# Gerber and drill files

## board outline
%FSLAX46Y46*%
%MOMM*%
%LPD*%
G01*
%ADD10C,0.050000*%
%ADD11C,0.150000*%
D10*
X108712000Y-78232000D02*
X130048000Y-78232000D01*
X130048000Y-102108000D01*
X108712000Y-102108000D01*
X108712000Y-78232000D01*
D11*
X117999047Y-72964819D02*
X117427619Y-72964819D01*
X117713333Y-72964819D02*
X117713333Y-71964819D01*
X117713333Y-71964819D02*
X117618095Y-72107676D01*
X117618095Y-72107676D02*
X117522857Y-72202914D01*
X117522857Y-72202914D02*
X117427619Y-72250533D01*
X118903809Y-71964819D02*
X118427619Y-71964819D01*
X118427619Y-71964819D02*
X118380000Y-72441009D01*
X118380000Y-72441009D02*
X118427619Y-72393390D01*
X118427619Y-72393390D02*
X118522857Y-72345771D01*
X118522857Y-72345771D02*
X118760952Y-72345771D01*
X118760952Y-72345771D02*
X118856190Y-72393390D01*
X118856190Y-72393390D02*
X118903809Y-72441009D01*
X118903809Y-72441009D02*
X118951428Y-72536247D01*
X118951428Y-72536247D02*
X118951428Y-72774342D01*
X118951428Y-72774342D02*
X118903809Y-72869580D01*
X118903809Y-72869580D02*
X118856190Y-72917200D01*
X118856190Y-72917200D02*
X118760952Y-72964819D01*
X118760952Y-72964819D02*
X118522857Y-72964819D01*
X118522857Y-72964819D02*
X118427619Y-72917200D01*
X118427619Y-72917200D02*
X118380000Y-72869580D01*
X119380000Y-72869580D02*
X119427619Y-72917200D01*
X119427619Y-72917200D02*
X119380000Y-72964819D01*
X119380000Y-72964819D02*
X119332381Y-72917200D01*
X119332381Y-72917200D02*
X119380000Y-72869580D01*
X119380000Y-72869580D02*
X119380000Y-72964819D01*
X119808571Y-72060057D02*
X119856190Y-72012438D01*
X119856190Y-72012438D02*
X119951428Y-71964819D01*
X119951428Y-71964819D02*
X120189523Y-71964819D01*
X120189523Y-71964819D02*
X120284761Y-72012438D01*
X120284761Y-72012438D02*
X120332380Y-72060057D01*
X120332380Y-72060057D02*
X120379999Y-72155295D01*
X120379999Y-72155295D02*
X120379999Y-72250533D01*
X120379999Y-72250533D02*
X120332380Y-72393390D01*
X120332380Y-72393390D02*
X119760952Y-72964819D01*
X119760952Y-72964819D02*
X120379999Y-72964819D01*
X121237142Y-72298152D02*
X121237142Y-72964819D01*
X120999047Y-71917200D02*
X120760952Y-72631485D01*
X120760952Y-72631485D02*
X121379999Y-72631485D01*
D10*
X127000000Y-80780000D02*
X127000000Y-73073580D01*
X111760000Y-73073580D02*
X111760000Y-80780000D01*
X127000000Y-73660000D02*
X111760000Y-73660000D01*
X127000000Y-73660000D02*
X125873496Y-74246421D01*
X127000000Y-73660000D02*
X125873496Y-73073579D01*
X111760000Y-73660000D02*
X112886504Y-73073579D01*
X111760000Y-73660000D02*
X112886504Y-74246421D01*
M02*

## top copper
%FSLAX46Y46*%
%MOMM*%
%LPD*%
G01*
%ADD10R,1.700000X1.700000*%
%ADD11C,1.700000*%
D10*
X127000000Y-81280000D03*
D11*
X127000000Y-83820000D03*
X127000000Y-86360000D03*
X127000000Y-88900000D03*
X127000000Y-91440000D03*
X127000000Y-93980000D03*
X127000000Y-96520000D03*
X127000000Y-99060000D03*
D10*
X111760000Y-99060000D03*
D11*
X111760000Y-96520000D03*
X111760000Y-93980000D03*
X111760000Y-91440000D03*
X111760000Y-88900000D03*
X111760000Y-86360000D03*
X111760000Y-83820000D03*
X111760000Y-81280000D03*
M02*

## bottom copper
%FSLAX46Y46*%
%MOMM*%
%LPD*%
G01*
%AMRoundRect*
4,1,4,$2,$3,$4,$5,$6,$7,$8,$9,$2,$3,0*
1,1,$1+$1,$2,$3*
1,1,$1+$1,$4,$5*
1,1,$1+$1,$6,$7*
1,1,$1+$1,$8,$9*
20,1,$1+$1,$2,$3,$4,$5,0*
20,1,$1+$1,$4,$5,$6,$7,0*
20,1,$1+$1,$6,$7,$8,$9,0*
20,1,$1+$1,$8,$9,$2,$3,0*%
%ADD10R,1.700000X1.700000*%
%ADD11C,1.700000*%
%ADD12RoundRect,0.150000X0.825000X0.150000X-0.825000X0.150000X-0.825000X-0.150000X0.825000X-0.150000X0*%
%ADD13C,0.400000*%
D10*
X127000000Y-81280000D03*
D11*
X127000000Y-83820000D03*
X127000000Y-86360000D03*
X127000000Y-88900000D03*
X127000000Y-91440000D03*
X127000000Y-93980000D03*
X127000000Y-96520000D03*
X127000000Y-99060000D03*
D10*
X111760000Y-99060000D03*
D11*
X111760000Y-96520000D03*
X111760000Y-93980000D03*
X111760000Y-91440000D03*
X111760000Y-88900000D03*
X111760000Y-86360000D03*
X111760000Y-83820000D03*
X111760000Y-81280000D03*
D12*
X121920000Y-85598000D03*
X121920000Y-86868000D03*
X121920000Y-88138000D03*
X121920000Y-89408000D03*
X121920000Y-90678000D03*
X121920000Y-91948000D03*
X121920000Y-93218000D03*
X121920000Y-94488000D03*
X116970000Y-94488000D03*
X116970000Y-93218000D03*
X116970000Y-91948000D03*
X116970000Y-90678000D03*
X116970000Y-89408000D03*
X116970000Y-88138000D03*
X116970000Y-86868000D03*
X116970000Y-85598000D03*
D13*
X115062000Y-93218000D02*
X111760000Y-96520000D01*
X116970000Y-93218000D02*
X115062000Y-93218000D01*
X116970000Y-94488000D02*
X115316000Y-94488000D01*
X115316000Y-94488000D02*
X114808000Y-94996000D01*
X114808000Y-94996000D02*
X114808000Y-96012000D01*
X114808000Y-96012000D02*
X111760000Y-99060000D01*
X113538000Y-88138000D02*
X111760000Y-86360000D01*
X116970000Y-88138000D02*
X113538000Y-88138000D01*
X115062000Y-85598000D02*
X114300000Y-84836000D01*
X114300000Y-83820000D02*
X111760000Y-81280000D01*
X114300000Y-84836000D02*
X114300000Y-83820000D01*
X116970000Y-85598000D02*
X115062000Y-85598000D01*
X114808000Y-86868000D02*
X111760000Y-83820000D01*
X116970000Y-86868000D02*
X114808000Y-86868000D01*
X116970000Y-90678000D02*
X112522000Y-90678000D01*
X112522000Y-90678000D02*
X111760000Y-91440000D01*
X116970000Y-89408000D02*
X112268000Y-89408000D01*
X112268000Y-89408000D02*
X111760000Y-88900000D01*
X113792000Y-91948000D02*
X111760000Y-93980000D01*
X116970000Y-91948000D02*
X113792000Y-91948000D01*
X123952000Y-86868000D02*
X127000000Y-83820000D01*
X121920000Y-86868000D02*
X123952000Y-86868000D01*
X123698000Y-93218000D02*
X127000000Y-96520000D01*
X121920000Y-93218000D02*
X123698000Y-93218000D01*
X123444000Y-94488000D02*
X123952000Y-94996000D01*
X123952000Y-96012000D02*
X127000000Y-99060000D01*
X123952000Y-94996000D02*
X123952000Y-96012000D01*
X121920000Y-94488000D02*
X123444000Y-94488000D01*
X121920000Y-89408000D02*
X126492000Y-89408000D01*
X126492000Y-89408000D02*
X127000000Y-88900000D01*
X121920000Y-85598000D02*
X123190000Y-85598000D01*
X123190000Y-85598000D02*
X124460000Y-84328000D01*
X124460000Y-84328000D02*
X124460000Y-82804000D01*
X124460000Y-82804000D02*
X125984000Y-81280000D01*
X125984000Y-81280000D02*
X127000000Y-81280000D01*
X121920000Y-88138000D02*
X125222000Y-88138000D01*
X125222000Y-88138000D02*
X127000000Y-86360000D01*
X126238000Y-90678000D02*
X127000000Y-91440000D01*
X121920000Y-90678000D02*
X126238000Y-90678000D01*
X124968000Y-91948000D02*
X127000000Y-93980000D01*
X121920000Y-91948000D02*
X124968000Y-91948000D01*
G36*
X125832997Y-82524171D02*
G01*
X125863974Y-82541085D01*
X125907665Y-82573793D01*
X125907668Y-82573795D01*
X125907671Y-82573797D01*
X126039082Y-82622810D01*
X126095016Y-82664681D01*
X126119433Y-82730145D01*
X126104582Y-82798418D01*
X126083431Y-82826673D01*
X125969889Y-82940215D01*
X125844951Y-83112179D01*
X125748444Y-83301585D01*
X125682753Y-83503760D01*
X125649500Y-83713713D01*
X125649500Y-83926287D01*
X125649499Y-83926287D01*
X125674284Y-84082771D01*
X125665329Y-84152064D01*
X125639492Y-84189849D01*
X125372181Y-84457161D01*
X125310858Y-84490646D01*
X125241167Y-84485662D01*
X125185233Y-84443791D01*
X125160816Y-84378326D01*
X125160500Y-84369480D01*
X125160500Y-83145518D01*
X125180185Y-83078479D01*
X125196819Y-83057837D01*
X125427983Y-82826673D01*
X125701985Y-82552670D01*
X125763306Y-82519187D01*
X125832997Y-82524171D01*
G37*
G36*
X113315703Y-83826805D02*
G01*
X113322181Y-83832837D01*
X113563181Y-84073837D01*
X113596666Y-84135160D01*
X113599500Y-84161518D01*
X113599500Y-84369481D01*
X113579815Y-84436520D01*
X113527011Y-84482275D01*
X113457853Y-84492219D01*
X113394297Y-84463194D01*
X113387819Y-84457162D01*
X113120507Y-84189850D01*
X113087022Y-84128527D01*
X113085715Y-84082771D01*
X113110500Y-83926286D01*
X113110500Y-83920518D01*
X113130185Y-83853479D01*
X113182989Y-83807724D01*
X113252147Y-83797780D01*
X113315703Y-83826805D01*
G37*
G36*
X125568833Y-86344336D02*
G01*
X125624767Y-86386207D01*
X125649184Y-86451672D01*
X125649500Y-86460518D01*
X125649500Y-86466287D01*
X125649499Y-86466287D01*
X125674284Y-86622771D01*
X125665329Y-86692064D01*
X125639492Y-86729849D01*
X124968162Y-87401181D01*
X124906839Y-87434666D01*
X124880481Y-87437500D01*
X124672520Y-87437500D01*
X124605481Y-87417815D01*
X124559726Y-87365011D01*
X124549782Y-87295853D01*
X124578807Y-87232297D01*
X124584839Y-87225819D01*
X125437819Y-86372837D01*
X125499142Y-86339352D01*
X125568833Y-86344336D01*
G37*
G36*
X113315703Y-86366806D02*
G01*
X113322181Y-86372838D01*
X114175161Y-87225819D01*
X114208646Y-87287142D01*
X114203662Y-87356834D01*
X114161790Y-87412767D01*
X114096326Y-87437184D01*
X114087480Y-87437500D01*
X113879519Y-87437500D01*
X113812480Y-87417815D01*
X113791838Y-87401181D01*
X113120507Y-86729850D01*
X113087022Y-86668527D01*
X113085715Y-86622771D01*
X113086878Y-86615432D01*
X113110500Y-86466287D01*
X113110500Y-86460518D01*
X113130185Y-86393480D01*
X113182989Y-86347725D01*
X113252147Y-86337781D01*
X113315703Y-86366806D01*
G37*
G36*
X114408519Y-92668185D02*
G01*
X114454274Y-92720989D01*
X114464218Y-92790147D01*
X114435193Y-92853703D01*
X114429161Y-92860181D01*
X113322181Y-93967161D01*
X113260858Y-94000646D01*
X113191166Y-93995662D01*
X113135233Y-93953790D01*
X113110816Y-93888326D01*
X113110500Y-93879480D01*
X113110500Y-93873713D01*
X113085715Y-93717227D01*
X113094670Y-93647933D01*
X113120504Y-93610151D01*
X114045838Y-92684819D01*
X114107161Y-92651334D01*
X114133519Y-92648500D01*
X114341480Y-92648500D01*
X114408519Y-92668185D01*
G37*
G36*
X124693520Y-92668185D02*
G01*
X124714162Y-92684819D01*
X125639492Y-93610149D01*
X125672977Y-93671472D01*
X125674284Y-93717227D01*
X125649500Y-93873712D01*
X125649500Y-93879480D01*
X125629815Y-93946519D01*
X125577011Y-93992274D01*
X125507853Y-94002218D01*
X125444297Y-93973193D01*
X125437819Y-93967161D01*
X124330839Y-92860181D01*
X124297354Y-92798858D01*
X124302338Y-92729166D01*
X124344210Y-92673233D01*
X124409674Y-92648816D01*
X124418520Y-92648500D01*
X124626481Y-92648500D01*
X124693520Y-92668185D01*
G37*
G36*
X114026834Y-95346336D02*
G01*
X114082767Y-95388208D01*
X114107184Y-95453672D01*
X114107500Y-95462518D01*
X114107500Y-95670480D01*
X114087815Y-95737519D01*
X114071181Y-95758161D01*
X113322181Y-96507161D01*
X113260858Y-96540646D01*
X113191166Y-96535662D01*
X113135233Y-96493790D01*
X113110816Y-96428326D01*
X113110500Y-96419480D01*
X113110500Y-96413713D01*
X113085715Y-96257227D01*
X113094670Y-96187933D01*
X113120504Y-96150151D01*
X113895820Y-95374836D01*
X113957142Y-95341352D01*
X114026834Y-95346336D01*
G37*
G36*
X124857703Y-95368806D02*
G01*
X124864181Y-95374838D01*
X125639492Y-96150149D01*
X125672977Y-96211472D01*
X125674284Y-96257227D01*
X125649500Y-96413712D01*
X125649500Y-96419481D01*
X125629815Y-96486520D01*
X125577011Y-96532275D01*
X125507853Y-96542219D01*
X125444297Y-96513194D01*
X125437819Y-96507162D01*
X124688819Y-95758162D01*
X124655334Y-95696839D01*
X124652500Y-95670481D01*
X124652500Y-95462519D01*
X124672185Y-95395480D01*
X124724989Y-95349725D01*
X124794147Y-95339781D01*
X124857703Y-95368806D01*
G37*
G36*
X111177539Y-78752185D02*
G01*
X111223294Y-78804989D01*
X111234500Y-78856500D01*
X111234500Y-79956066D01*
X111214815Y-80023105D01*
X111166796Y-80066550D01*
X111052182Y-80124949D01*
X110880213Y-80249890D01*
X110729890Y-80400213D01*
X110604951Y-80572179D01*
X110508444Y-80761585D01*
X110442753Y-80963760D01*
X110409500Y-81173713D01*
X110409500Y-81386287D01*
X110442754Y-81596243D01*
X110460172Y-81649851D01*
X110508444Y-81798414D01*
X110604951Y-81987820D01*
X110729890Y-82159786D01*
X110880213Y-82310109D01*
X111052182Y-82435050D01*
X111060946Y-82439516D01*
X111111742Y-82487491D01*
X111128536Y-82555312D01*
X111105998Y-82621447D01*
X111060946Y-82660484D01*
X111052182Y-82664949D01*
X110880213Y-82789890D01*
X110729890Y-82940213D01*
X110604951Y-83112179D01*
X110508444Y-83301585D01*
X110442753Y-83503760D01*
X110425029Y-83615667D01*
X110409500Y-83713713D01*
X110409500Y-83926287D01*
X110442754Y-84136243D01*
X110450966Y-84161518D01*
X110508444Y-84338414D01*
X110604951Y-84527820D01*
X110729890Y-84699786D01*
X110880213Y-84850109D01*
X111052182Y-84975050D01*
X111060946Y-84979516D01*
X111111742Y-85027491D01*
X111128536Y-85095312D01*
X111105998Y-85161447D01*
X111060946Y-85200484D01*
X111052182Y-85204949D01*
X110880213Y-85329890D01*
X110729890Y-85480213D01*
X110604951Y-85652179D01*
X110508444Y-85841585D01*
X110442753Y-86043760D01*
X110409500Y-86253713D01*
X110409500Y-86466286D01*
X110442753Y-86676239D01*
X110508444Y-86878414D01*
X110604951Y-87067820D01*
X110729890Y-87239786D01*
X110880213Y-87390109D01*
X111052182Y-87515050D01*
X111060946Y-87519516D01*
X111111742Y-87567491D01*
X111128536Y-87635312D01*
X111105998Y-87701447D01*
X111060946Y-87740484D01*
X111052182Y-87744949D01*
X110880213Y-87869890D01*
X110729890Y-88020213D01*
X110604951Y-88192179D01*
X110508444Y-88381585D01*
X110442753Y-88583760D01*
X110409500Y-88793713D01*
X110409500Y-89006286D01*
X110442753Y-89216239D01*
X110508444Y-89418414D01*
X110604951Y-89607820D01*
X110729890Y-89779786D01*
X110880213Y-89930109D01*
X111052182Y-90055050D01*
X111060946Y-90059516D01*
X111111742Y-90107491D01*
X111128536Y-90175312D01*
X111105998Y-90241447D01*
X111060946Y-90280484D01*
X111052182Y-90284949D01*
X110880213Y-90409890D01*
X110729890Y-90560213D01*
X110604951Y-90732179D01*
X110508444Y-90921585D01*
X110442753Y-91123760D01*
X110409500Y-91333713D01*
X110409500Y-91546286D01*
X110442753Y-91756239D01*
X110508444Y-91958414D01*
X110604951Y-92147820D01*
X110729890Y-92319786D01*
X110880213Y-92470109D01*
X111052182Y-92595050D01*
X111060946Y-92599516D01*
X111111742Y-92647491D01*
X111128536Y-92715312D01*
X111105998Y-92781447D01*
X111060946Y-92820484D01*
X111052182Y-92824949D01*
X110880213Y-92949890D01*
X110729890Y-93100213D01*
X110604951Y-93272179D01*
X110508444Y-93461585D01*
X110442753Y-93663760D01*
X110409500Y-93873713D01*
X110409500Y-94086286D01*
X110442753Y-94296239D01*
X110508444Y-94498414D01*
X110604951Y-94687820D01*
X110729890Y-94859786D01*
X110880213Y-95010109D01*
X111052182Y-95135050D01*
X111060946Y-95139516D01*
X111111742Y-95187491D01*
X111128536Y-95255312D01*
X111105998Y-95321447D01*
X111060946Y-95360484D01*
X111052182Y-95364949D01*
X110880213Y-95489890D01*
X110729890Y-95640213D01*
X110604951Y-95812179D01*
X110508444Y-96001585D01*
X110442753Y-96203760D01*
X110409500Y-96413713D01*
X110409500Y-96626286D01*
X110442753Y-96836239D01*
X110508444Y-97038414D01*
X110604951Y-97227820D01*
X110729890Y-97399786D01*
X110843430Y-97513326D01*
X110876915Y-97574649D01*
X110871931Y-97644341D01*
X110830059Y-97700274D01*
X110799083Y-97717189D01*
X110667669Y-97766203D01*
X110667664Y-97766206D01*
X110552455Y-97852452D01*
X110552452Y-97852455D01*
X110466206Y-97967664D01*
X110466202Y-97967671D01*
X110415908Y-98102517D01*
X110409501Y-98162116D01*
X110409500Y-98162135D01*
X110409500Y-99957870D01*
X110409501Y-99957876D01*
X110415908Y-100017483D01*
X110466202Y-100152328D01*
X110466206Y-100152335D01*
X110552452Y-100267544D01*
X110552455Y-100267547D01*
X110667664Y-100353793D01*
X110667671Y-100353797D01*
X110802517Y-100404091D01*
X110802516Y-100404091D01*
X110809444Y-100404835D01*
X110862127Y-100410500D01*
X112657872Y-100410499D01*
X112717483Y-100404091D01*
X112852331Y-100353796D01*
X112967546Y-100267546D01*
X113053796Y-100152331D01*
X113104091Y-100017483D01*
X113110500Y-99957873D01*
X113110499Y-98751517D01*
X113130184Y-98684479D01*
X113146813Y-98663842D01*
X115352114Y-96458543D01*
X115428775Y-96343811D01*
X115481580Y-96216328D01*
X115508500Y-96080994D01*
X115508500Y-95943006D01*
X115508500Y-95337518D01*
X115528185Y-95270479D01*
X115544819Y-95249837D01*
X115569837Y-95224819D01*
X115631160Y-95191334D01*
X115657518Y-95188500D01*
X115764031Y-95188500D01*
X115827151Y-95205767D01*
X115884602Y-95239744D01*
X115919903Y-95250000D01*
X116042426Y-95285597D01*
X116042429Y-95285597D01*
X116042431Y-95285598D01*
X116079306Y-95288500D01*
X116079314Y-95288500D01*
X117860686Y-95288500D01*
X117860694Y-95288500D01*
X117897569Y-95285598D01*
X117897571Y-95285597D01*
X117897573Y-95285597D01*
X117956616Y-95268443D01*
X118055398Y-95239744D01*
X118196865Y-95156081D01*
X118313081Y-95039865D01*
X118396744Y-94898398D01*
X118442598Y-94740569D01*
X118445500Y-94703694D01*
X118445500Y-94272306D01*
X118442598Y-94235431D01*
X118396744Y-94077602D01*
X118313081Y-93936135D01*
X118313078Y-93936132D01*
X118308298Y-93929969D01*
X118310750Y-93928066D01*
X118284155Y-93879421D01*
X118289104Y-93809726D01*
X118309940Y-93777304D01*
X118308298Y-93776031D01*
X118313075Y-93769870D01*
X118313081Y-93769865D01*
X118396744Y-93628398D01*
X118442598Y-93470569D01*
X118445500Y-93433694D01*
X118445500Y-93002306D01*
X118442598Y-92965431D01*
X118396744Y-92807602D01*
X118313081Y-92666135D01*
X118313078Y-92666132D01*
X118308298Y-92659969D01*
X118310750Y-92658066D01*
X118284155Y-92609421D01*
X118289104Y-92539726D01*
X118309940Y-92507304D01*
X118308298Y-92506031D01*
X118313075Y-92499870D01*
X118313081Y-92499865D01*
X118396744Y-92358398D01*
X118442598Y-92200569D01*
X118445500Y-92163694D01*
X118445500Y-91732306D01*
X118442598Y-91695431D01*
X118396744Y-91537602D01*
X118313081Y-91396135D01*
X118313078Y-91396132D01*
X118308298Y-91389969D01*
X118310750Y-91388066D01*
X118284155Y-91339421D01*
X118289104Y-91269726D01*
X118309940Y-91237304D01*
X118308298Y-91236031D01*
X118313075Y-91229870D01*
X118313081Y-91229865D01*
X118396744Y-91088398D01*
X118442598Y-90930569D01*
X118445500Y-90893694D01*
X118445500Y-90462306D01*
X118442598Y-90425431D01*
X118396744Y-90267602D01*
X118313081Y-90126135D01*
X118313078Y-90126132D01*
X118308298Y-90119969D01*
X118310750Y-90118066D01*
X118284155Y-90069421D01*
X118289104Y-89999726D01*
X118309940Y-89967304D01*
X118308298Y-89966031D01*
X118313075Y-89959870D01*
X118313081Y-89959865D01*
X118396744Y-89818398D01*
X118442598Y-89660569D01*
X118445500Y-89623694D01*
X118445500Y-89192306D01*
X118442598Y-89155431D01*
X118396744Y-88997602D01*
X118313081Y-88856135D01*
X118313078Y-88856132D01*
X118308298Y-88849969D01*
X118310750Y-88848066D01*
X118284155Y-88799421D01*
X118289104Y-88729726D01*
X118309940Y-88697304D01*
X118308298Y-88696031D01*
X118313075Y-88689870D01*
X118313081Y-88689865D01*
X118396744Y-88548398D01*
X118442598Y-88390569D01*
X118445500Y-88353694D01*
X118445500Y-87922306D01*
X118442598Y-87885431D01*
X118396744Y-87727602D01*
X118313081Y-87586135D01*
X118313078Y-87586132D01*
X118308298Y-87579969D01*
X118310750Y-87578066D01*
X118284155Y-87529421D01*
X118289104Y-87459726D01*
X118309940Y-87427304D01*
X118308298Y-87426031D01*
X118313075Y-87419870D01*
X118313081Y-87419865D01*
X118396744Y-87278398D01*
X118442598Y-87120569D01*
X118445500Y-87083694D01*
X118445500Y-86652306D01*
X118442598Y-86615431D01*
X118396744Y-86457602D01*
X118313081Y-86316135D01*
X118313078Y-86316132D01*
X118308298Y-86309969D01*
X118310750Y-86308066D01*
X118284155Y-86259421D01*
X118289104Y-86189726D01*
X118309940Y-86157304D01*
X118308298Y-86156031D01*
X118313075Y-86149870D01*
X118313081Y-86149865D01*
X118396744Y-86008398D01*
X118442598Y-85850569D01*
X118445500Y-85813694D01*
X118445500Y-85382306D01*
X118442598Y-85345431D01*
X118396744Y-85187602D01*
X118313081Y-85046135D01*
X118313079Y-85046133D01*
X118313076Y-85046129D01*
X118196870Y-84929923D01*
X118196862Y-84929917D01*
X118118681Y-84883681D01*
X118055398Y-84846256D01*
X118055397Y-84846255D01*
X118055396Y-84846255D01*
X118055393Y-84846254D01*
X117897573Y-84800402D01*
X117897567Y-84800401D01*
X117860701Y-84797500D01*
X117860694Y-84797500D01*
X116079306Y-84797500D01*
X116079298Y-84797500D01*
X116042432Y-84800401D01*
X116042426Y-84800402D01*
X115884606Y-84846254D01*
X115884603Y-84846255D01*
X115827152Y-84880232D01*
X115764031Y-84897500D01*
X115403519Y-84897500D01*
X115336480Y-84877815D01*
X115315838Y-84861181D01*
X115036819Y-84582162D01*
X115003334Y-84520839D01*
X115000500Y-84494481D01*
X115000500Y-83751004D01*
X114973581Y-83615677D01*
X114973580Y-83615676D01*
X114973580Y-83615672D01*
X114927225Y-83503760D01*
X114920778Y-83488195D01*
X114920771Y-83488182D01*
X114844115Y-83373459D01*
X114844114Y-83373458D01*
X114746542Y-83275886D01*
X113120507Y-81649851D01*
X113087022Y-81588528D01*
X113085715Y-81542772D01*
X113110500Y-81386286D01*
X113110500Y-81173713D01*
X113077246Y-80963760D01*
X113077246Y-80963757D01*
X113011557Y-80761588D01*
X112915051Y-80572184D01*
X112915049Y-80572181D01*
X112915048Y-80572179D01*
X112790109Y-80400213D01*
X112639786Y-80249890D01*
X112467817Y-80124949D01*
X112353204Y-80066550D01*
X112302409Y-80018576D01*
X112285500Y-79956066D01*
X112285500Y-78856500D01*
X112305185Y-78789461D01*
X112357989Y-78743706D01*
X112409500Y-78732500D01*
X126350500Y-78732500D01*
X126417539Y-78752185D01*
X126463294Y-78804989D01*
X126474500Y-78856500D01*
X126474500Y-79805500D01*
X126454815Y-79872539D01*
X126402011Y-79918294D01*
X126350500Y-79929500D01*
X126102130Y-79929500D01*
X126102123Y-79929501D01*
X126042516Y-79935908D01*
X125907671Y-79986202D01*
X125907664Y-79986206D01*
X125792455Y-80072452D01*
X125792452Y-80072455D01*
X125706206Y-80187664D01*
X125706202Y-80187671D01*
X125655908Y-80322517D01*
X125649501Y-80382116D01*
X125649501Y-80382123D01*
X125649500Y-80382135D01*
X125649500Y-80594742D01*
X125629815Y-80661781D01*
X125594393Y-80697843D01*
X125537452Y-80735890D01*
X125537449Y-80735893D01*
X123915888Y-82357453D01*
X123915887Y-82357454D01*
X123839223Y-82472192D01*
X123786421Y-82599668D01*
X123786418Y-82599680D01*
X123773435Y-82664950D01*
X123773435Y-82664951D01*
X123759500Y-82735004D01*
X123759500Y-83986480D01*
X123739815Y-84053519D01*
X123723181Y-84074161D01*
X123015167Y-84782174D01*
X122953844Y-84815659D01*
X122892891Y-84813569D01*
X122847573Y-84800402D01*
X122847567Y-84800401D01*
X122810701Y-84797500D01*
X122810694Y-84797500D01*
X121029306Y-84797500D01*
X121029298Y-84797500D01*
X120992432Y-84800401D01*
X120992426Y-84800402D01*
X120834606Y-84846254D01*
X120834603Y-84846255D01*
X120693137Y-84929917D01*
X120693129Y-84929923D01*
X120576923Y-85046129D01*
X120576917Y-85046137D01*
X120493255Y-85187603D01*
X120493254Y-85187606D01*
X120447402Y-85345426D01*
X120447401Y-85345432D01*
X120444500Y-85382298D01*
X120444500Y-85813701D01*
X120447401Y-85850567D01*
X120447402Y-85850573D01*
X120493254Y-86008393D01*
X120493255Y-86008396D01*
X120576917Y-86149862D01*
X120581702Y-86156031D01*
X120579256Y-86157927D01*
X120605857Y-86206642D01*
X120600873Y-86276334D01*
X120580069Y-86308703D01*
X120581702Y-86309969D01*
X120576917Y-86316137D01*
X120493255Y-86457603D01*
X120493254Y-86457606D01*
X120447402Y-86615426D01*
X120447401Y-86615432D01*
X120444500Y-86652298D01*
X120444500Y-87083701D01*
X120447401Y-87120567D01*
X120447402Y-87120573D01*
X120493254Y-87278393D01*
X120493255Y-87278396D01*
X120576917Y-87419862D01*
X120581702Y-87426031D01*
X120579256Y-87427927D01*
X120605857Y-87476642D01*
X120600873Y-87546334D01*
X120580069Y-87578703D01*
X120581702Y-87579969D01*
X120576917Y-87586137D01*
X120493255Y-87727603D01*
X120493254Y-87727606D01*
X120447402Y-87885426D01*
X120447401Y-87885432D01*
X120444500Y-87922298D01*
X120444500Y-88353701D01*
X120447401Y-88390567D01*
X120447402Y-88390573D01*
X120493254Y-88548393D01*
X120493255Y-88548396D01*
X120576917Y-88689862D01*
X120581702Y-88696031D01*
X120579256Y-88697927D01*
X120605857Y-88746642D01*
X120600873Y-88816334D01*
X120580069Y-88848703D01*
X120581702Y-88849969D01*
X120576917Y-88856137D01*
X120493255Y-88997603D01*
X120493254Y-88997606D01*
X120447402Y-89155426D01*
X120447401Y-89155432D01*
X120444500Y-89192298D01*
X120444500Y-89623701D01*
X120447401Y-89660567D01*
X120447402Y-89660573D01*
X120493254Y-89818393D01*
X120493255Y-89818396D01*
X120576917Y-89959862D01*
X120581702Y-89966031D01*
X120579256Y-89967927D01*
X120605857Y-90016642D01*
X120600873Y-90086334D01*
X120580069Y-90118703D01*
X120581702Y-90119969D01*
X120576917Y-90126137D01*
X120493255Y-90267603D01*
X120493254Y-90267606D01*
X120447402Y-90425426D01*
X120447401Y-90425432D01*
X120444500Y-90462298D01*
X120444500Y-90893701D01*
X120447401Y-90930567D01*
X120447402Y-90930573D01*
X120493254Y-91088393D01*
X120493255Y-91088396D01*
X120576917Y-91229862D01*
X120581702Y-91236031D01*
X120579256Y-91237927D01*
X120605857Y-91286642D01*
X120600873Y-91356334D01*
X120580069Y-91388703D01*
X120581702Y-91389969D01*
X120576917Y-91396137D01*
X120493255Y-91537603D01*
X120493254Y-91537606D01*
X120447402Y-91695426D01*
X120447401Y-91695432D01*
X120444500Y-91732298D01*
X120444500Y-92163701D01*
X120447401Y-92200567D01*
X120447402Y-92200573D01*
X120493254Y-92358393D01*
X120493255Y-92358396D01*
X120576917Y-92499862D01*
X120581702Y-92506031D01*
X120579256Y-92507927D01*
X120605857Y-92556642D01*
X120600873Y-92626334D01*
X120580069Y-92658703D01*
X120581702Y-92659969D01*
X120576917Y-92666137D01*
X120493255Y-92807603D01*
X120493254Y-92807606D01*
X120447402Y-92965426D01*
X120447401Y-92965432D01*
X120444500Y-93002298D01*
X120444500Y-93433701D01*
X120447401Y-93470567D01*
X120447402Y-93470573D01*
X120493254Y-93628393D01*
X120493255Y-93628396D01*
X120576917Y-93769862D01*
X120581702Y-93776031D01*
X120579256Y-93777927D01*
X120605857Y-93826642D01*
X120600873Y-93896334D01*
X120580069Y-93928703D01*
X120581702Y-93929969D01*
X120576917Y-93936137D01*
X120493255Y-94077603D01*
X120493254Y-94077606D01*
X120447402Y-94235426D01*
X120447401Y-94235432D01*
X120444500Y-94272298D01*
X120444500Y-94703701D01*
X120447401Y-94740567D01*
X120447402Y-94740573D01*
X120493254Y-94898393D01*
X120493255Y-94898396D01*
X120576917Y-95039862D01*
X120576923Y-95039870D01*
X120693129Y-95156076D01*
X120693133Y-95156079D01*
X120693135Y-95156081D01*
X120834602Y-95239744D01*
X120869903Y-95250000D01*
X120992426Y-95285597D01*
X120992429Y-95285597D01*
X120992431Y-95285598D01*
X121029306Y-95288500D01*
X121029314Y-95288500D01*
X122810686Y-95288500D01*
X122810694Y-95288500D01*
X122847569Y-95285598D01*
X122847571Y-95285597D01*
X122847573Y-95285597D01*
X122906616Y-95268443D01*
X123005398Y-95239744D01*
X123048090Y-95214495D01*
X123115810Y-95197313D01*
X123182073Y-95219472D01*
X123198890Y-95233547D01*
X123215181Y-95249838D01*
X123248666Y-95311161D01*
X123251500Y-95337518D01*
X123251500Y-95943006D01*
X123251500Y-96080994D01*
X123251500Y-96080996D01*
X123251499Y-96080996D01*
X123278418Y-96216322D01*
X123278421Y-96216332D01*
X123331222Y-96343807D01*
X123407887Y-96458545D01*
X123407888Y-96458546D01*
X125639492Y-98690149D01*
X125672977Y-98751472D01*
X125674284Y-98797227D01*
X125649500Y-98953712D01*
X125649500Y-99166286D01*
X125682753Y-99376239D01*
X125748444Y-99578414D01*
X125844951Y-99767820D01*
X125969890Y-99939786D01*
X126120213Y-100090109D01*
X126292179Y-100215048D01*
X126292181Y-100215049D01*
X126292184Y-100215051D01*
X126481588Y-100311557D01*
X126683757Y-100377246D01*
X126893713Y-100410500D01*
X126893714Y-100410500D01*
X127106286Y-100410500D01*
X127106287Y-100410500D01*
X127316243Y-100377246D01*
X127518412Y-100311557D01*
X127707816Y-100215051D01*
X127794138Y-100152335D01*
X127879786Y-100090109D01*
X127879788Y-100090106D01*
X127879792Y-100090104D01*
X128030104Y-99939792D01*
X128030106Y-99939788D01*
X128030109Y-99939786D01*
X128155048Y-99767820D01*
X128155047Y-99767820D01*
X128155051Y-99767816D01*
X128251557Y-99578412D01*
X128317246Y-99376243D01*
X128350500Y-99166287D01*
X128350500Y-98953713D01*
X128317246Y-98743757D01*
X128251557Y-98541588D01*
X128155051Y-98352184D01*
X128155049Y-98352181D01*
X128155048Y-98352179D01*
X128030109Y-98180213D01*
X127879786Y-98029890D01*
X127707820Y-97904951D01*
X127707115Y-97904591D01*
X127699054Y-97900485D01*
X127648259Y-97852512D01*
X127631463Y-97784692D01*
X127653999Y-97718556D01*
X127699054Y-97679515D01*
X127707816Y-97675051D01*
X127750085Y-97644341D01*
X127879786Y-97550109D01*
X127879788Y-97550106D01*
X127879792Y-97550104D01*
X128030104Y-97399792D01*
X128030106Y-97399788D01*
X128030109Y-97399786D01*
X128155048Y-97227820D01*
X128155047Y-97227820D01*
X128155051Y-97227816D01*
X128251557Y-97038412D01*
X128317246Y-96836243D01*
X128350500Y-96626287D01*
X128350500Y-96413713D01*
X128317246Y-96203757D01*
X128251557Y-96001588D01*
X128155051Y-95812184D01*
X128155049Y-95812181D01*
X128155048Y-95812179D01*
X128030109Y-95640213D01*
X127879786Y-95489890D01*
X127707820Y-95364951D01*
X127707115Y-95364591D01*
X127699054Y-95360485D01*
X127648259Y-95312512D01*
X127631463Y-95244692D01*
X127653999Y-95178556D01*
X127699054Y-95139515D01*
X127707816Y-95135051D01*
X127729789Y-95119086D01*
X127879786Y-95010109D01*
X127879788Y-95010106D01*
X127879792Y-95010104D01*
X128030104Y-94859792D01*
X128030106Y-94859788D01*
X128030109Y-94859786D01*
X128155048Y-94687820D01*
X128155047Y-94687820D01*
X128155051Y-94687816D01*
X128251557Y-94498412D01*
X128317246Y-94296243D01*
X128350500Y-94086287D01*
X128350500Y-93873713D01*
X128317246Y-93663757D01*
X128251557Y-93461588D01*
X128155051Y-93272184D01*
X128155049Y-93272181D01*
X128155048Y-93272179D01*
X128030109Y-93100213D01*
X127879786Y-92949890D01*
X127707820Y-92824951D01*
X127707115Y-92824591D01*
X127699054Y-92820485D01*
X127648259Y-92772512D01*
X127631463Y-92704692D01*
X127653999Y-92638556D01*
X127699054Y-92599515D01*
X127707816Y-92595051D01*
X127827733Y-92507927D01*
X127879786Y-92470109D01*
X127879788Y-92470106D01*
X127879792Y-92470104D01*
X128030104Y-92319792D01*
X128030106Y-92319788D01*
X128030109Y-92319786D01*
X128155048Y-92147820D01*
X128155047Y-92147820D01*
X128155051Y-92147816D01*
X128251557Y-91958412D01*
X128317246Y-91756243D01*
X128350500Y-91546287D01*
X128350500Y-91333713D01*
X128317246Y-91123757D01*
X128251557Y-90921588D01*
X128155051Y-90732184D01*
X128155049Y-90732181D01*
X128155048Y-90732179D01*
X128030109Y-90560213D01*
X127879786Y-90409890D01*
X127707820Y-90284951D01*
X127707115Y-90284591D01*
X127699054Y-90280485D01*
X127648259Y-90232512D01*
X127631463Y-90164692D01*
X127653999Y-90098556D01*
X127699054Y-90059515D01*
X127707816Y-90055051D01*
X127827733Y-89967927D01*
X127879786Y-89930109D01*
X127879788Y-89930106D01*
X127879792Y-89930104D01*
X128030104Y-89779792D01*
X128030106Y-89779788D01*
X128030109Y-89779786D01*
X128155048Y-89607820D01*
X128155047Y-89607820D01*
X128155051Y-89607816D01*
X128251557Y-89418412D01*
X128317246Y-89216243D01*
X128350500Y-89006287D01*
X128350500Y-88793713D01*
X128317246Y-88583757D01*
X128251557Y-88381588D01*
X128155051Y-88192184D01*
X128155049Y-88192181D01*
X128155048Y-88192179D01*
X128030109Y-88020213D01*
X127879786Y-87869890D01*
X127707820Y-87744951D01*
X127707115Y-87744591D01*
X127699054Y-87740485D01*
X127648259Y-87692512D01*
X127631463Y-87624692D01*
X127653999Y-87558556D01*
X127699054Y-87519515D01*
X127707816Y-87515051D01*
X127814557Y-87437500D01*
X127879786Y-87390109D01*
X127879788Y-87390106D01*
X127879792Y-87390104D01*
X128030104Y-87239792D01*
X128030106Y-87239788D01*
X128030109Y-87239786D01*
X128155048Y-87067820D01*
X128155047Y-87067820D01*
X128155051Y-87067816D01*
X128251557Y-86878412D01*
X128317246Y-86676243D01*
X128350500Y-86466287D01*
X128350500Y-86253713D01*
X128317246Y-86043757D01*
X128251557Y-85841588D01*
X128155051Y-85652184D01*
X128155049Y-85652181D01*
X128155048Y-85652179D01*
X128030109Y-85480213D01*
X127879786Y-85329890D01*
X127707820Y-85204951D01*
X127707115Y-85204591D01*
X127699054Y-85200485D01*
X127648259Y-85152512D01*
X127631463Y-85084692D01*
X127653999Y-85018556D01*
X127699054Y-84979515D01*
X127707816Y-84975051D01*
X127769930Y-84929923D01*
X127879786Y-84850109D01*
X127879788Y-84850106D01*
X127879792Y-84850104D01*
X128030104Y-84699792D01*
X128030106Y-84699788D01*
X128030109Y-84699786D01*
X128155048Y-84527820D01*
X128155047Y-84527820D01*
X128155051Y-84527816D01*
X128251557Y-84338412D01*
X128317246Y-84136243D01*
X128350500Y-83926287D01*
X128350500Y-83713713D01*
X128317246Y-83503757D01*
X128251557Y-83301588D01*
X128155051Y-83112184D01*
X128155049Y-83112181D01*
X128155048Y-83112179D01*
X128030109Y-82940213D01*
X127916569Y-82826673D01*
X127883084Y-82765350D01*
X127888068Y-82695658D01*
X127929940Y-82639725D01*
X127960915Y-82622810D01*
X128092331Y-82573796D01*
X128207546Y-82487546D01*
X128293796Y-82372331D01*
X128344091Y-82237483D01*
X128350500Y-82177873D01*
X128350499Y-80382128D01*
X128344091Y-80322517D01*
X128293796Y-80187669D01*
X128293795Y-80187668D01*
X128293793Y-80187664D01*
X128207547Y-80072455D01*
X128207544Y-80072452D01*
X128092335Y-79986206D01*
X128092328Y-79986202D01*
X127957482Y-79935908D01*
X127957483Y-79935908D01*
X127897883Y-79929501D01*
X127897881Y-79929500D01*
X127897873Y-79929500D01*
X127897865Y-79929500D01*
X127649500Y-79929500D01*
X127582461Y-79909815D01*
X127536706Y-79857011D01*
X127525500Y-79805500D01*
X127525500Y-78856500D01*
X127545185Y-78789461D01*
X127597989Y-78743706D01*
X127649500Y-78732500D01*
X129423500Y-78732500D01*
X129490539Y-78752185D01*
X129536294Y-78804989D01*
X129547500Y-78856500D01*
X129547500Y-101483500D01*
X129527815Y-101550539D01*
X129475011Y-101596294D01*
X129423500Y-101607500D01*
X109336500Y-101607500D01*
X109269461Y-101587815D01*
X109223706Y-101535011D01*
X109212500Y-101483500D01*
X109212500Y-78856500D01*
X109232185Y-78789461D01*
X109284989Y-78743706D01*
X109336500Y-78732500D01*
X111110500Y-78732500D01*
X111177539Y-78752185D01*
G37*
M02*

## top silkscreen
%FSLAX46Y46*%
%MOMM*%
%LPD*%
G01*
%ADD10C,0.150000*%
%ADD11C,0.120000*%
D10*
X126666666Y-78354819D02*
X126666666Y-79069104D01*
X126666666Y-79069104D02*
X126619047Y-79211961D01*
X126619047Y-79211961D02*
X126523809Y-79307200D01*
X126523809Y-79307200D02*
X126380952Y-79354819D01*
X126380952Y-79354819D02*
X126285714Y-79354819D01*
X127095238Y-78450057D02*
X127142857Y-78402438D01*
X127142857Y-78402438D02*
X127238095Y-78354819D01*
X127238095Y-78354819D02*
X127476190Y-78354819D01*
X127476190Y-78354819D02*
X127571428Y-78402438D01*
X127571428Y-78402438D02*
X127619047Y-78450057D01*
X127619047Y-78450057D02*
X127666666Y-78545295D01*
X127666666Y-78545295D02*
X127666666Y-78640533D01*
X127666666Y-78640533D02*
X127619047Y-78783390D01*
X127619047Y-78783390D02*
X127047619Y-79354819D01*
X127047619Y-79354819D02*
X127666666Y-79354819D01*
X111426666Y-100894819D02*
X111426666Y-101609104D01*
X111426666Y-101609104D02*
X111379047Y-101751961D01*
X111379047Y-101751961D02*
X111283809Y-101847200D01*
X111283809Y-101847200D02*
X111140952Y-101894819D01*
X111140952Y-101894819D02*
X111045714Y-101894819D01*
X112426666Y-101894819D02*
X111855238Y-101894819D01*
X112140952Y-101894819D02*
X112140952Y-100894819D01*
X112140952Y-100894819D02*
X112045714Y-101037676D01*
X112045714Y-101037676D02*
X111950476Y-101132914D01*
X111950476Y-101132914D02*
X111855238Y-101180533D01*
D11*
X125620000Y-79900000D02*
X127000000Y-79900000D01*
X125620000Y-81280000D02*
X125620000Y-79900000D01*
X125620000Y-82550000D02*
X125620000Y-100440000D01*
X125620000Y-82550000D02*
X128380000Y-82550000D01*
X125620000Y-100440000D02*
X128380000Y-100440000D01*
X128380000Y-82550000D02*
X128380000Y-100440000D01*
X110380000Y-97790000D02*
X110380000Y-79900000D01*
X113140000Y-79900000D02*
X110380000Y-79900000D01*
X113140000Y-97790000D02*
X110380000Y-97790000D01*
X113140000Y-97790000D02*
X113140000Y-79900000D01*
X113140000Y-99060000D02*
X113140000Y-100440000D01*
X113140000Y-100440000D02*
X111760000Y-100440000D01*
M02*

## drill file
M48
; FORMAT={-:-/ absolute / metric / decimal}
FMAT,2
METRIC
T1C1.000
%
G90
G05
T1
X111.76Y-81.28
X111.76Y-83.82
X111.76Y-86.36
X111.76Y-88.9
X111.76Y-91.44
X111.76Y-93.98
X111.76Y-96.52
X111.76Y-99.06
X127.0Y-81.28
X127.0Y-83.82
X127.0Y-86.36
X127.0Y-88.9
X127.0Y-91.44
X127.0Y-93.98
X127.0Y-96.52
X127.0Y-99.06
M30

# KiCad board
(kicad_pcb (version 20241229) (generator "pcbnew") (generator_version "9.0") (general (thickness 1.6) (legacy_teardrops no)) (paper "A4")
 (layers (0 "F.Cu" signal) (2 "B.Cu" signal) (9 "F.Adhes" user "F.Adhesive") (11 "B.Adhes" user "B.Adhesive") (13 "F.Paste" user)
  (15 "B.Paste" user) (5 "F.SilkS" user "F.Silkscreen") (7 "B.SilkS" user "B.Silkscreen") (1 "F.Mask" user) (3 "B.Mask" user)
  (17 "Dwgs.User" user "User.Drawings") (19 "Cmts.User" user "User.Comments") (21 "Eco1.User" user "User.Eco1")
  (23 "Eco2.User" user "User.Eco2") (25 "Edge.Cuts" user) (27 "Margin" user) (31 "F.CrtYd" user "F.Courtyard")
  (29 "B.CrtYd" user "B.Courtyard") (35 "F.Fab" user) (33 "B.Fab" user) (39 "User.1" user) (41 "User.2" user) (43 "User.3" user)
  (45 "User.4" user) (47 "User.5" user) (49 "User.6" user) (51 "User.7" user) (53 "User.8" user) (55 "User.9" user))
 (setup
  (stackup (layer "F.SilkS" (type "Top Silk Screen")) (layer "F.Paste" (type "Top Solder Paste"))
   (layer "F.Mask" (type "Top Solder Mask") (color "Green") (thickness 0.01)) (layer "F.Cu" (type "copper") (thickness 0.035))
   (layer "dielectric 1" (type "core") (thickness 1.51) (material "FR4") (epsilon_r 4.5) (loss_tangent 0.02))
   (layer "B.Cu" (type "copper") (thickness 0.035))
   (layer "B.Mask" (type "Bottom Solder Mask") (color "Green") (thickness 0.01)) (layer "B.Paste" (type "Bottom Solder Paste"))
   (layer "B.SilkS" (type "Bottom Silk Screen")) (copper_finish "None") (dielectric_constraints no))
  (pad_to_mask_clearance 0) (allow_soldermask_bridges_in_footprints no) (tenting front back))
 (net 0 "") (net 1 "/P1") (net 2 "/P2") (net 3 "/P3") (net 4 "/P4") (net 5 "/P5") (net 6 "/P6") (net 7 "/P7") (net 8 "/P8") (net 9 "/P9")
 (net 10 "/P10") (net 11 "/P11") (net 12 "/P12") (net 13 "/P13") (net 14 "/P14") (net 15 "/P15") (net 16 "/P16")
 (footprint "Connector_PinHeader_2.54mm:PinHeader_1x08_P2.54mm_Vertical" (layer "F.Cu") (at 127 81.28)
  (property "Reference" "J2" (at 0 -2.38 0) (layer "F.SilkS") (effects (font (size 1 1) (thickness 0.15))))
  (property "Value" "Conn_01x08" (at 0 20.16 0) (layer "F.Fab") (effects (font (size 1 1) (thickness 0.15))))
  (fp_line (start -1.38 -1.38) (end 0 -1.38) (stroke (width 0.12) (type solid)) (layer "F.SilkS"))
  (fp_line (start -1.38 0) (end -1.38 -1.38) (stroke (width 0.12) (type solid)) (layer "F.SilkS"))
  (fp_line (start -1.38 1.27) (end -1.38 19.16) (stroke (width 0.12) (type solid)) (layer "F.SilkS"))
  (fp_line (start -1.38 1.27) (end 1.38 1.27) (stroke (width 0.12) (type solid)) (layer "F.SilkS"))
  (fp_line (start -1.38 19.16) (end 1.38 19.16) (stroke (width 0.12) (type solid)) (layer "F.SilkS"))
  (fp_line (start 1.38 1.27) (end 1.38 19.16) (stroke (width 0.12) (type solid)) (layer "F.SilkS"))
  (pad "1" thru_hole rect (at 0 0) (size 1.7 1.7) (drill 1) (layers "*.Cu" "*.Mask") (remove_unused_layers no) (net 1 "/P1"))
  (pad "2" thru_hole circle (at 0 2.54) (size 1.7 1.7) (drill 1) (layers "*.Cu" "*.Mask") (remove_unused_layers no) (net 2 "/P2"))
  (pad "3" thru_hole circle (at 0 5.08) (size 1.7 1.7) (drill 1) (layers "*.Cu" "*.Mask") (remove_unused_layers no) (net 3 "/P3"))
  (pad "4" thru_hole circle (at 0 7.62) (size 1.7 1.7) (drill 1) (layers "*.Cu" "*.Mask") (remove_unused_layers no) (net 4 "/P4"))
  (pad "5" thru_hole circle (at 0 10.16) (size 1.7 1.7) (drill 1) (layers "*.Cu" "*.Mask") (remove_unused_layers no) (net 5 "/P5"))
  (pad "6" thru_hole circle (at 0 12.7) (size 1.7 1.7) (drill 1) (layers "*.Cu" "*.Mask") (remove_unused_layers no) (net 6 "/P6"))
  (pad "7" thru_hole circle (at 0 15.24) (size 1.7 1.7) (drill 1) (layers "*.Cu" "*.Mask") (remove_unused_layers no) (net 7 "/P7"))
  (pad "8" thru_hole circle (at 0 17.78) (size 1.7 1.7) (drill 1) (layers "*.Cu" "*.Mask") (remove_unused_layers no) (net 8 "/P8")))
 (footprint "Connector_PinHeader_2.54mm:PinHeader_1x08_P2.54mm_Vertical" (layer "F.Cu") (at 111.76 99.06 180)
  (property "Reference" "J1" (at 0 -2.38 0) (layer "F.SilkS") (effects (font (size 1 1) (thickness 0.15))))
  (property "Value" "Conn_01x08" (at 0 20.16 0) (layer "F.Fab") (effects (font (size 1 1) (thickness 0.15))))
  (fp_line (start 1.38 1.27) (end 1.38 19.16) (stroke (width 0.12) (type solid)) (layer "F.SilkS"))
  (fp_line (start -1.38 19.16) (end 1.38 19.16) (stroke (width 0.12) (type solid)) (layer "F.SilkS"))
  (fp_line (start -1.38 1.27) (end 1.38 1.27) (stroke (width 0.12) (type solid)) (layer "F.SilkS"))
  (fp_line (start -1.38 1.27) (end -1.38 19.16) (stroke (width 0.12) (type solid)) (layer "F.SilkS"))
  (fp_line (start -1.38 0) (end -1.38 -1.38) (stroke (width 0.12) (type solid)) (layer "F.SilkS"))
  (fp_line (start -1.38 -1.38) (end 0 -1.38) (stroke (width 0.12) (type solid)) (layer "F.SilkS"))
  (pad "1" thru_hole rect (at 0 0 180) (size 1.7 1.7) (drill 1) (layers "*.Cu" "*.Mask") (remove_unused_layers no) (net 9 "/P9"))
  (pad "2" thru_hole circle (at 0 2.54 180) (size 1.7 1.7) (drill 1) (layers "*.Cu" "*.Mask") (remove_unused_layers no) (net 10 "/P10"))
  (pad "3" thru_hole circle (at 0 5.08 180) (size 1.7 1.7) (drill 1) (layers "*.Cu" "*.Mask") (remove_unused_layers no) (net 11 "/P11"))
  (pad "4" thru_hole circle (at 0 7.62 180) (size 1.7 1.7) (drill 1) (layers "*.Cu" "*.Mask") (remove_unused_layers no) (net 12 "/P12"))
  (pad "5" thru_hole circle (at 0 10.16 180) (size 1.7 1.7) (drill 1) (layers "*.Cu" "*.Mask") (remove_unused_layers no) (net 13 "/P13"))
  (pad "6" thru_hole circle (at 0 12.7 180) (size 1.7 1.7) (drill 1) (layers "*.Cu" "*.Mask") (remove_unused_layers no) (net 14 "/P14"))
  (pad "7" thru_hole circle (at 0 15.24 180) (size 1.7 1.7) (drill 1) (layers "*.Cu" "*.Mask") (remove_unused_layers no) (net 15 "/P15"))
  (pad "8" thru_hole circle (at 0 17.78 180) (size 1.7 1.7) (drill 1) (layers "*.Cu" "*.Mask") (remove_unused_layers no) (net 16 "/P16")))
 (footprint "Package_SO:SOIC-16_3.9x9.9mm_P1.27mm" (layer "B.Cu") (at 119.445 90.043 180)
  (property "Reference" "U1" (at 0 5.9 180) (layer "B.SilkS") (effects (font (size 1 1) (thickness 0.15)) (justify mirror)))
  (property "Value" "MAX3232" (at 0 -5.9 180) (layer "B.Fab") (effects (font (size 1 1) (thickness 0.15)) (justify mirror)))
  (pad "1" smd roundrect (at -2.475 4.445 180) (size 1.95 0.6) (layers "B.Cu" "B.Mask" "B.Paste") (roundrect_rratio 0.25) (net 1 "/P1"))
  (pad "2" smd roundrect (at -2.475 3.175 180) (size 1.95 0.6) (layers "B.Cu" "B.Mask" "B.Paste") (roundrect_rratio 0.25) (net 2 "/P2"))
  (pad "3" smd roundrect (at -2.475 1.905 180) (size 1.95 0.6) (layers "B.Cu" "B.Mask" "B.Paste") (roundrect_rratio 0.25) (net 3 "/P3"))
  (pad "4" smd roundrect (at -2.475 0.635 180) (size 1.95 0.6) (layers "B.Cu" "B.Mask" "B.Paste") (roundrect_rratio 0.25) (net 4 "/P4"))
  (pad "5" smd roundrect (at -2.475 -0.635 180) (size 1.95 0.6) (layers "B.Cu" "B.Mask" "B.Paste") (roundrect_rratio 0.25) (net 5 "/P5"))
  (pad "6" smd roundrect (at -2.475 -1.905 180) (size 1.95 0.6) (layers "B.Cu" "B.Mask" "B.Paste") (roundrect_rratio 0.25) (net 6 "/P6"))
  (pad "7" smd roundrect (at -2.475 -3.175 180) (size 1.95 0.6) (layers "B.Cu" "B.Mask" "B.Paste") (roundrect_rratio 0.25) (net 7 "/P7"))
  (pad "8" smd roundrect (at -2.475 -4.445 180) (size 1.95 0.6) (layers "B.Cu" "B.Mask" "B.Paste") (roundrect_rratio 0.25) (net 8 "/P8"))
  (pad "9" smd roundrect (at 2.475 -4.445 180) (size 1.95 0.6) (layers "B.Cu" "B.Mask" "B.Paste") (roundrect_rratio 0.25) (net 9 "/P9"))
  (pad "10" smd roundrect (at 2.475 -3.175 180) (size 1.95 0.6) (layers "B.Cu" "B.Mask" "B.Paste") (roundrect_rratio 0.25) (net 10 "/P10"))
  (pad "11" smd roundrect (at 2.475 -1.905 180) (size 1.95 0.6) (layers "B.Cu" "B.Mask" "B.Paste") (roundrect_rratio 0.25) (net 11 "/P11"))
  (pad "12" smd roundrect (at 2.475 -0.635 180) (size 1.95 0.6) (layers "B.Cu" "B.Mask" "B.Paste") (roundrect_rratio 0.25) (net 12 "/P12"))
  (pad "13" smd roundrect (at 2.475 0.635 180) (size 1.95 0.6) (layers "B.Cu" "B.Mask" "B.Paste") (roundrect_rratio 0.25) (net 13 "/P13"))
  (pad "14" smd roundrect (at 2.475 1.905 180) (size 1.95 0.6) (layers "B.Cu" "B.Mask" "B.Paste") (roundrect_rratio 0.25) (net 14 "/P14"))
  (pad "15" smd roundrect (at 2.475 3.175 180) (size 1.95 0.6) (layers "B.Cu" "B.Mask" "B.Paste") (roundrect_rratio 0.25) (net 15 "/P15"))
  (pad "16" smd roundrect (at 2.475 4.445 180) (size 1.95 0.6) (layers "B.Cu" "B.Mask" "B.Paste") (roundrect_rratio 0.25) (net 16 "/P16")))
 (gr_rect (start 108.712 78.232) (end 130.048 102.108) (stroke (width 0.05) (type default)) (fill no) (layer "Edge.Cuts"))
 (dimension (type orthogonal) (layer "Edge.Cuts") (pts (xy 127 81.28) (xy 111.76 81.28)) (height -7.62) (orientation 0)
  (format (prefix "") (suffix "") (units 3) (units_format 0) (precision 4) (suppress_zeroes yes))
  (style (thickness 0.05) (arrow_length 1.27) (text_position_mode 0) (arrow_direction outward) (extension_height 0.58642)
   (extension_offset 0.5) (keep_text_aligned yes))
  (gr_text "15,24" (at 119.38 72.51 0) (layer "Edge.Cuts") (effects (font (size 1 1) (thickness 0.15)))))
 (segment (start 115.062 93.218) (end 111.76 96.52) (width 0.4) (layer "B.Cu") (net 10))
 (segment (start 116.97 93.218) (end 115.062 93.218) (width 0.4) (layer "B.Cu") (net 10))
 (segment (start 116.97 94.488) (end 115.316 94.488) (width 0.4) (layer "B.Cu") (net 9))
 (segment (start 115.316 94.488) (end 114.808 94.996) (width 0.4) (layer "B.Cu") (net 9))
 (segment (start 114.808 94.996) (end 114.808 96.012) (width 0.4) (layer "B.Cu") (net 9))
 (segment (start 114.808 96.012) (end 111.76 99.06) (width 0.4) (layer "B.Cu") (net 9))
 (segment (start 113.538 88.138) (end 111.76 86.36) (width 0.4) (layer "B.Cu") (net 14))
 (segment (start 116.97 88.138) (end 113.538 88.138) (width 0.4) (layer "B.Cu") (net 14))
 (segment (start 115.062 85.598) (end 114.3 84.836) (width 0.4) (layer "B.Cu") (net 16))
 (segment (start 114.3 83.82) (end 111.76 81.28) (width 0.4) (layer "B.Cu") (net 16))
 (segment (start 114.3 84.836) (end 114.3 83.82) (width 0.4) (layer "B.Cu") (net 16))
 (segment (start 116.97 85.598) (end 115.062 85.598) (width 0.4) (layer "B.Cu") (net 16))
 (segment (start 114.808 86.868) (end 111.76 83.82) (width 0.4) (layer "B.Cu") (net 15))
 (segment (start 116.97 86.868) (end 114.808 86.868) (width 0.4) (layer "B.Cu") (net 15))
 (segment (start 116.97 90.678) (end 112.522 90.678) (width 0.4) (layer "B.Cu") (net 12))
 (segment (start 112.522 90.678) (end 111.76 91.44) (width 0.4) (layer "B.Cu") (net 12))
 (segment (start 116.97 89.408) (end 112.268 89.408) (width 0.4) (layer "B.Cu") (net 13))
 (segment (start 112.268 89.408) (end 111.76 88.9) (width 0.4) (layer "B.Cu") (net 13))
 (segment (start 113.792 91.948) (end 111.76 93.98) (width 0.4) (layer "B.Cu") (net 11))
 (segment (start 116.97 91.948) (end 113.792 91.948) (width 0.4) (layer "B.Cu") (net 11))
 (segment (start 123.952 86.868) (end 127 83.82) (width 0.4) (layer "B.Cu") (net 2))
 (segment (start 121.92 86.868) (end 123.952 86.868) (width 0.4) (layer "B.Cu") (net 2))
 (segment (start 123.698 93.218) (end 127 96.52) (width 0.4) (layer "B.Cu") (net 7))
 (segment (start 121.92 93.218) (end 123.698 93.218) (width 0.4) (layer "B.Cu") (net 7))
 (segment (start 123.444 94.488) (end 123.952 94.996) (width 0.4) (layer "B.Cu") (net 8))
 (segment (start 123.952 96.012) (end 127 99.06) (width 0.4) (layer "B.Cu") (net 8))
 (segment (start 123.952 94.996) (end 123.952 96.012) (width 0.4) (layer "B.Cu") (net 8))
 (segment (start 121.92 94.488) (end 123.444 94.488) (width 0.4) (layer "B.Cu") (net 8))
 (segment (start 121.92 89.408) (end 126.492 89.408) (width 0.4) (layer "B.Cu") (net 4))
 (segment (start 126.492 89.408) (end 127 88.9) (width 0.4) (layer "B.Cu") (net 4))
 (segment (start 121.92 85.598) (end 123.19 85.598) (width 0.4) (layer "B.Cu") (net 1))
 (segment (start 123.19 85.598) (end 124.46 84.328) (width 0.4) (layer "B.Cu") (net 1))
 (segment (start 124.46 84.328) (end 124.46 82.804) (width 0.4) (layer "B.Cu") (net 1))
 (segment (start 124.46 82.804) (end 125.984 81.28) (width 0.4) (layer "B.Cu") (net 1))
 (segment (start 125.984 81.28) (end 127 81.28) (width 0.4) (layer "B.Cu") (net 1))
 (segment (start 121.92 88.138) (end 125.222 88.138) (width 0.4) (layer "B.Cu") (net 3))
 (segment (start 125.222 88.138) (end 127 86.36) (width 0.4) (layer "B.Cu") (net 3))
 (segment (start 126.238 90.678) (end 127 91.44) (width 0.4) (layer "B.Cu") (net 5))
 (segment (start 121.92 90.678) (end 126.238 90.678) (width 0.4) (layer "B.Cu") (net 5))
 (segment (start 124.968 91.948) (end 127 93.98) (width 0.4) (layer "B.Cu") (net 6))
 (segment (start 121.92 91.948) (end 124.968 91.948) (width 0.4) (layer "B.Cu") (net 6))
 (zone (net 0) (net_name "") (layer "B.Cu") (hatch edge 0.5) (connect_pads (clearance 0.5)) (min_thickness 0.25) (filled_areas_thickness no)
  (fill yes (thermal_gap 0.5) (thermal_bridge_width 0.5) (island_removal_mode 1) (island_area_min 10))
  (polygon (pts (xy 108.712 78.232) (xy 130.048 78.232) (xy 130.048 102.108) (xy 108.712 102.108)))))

